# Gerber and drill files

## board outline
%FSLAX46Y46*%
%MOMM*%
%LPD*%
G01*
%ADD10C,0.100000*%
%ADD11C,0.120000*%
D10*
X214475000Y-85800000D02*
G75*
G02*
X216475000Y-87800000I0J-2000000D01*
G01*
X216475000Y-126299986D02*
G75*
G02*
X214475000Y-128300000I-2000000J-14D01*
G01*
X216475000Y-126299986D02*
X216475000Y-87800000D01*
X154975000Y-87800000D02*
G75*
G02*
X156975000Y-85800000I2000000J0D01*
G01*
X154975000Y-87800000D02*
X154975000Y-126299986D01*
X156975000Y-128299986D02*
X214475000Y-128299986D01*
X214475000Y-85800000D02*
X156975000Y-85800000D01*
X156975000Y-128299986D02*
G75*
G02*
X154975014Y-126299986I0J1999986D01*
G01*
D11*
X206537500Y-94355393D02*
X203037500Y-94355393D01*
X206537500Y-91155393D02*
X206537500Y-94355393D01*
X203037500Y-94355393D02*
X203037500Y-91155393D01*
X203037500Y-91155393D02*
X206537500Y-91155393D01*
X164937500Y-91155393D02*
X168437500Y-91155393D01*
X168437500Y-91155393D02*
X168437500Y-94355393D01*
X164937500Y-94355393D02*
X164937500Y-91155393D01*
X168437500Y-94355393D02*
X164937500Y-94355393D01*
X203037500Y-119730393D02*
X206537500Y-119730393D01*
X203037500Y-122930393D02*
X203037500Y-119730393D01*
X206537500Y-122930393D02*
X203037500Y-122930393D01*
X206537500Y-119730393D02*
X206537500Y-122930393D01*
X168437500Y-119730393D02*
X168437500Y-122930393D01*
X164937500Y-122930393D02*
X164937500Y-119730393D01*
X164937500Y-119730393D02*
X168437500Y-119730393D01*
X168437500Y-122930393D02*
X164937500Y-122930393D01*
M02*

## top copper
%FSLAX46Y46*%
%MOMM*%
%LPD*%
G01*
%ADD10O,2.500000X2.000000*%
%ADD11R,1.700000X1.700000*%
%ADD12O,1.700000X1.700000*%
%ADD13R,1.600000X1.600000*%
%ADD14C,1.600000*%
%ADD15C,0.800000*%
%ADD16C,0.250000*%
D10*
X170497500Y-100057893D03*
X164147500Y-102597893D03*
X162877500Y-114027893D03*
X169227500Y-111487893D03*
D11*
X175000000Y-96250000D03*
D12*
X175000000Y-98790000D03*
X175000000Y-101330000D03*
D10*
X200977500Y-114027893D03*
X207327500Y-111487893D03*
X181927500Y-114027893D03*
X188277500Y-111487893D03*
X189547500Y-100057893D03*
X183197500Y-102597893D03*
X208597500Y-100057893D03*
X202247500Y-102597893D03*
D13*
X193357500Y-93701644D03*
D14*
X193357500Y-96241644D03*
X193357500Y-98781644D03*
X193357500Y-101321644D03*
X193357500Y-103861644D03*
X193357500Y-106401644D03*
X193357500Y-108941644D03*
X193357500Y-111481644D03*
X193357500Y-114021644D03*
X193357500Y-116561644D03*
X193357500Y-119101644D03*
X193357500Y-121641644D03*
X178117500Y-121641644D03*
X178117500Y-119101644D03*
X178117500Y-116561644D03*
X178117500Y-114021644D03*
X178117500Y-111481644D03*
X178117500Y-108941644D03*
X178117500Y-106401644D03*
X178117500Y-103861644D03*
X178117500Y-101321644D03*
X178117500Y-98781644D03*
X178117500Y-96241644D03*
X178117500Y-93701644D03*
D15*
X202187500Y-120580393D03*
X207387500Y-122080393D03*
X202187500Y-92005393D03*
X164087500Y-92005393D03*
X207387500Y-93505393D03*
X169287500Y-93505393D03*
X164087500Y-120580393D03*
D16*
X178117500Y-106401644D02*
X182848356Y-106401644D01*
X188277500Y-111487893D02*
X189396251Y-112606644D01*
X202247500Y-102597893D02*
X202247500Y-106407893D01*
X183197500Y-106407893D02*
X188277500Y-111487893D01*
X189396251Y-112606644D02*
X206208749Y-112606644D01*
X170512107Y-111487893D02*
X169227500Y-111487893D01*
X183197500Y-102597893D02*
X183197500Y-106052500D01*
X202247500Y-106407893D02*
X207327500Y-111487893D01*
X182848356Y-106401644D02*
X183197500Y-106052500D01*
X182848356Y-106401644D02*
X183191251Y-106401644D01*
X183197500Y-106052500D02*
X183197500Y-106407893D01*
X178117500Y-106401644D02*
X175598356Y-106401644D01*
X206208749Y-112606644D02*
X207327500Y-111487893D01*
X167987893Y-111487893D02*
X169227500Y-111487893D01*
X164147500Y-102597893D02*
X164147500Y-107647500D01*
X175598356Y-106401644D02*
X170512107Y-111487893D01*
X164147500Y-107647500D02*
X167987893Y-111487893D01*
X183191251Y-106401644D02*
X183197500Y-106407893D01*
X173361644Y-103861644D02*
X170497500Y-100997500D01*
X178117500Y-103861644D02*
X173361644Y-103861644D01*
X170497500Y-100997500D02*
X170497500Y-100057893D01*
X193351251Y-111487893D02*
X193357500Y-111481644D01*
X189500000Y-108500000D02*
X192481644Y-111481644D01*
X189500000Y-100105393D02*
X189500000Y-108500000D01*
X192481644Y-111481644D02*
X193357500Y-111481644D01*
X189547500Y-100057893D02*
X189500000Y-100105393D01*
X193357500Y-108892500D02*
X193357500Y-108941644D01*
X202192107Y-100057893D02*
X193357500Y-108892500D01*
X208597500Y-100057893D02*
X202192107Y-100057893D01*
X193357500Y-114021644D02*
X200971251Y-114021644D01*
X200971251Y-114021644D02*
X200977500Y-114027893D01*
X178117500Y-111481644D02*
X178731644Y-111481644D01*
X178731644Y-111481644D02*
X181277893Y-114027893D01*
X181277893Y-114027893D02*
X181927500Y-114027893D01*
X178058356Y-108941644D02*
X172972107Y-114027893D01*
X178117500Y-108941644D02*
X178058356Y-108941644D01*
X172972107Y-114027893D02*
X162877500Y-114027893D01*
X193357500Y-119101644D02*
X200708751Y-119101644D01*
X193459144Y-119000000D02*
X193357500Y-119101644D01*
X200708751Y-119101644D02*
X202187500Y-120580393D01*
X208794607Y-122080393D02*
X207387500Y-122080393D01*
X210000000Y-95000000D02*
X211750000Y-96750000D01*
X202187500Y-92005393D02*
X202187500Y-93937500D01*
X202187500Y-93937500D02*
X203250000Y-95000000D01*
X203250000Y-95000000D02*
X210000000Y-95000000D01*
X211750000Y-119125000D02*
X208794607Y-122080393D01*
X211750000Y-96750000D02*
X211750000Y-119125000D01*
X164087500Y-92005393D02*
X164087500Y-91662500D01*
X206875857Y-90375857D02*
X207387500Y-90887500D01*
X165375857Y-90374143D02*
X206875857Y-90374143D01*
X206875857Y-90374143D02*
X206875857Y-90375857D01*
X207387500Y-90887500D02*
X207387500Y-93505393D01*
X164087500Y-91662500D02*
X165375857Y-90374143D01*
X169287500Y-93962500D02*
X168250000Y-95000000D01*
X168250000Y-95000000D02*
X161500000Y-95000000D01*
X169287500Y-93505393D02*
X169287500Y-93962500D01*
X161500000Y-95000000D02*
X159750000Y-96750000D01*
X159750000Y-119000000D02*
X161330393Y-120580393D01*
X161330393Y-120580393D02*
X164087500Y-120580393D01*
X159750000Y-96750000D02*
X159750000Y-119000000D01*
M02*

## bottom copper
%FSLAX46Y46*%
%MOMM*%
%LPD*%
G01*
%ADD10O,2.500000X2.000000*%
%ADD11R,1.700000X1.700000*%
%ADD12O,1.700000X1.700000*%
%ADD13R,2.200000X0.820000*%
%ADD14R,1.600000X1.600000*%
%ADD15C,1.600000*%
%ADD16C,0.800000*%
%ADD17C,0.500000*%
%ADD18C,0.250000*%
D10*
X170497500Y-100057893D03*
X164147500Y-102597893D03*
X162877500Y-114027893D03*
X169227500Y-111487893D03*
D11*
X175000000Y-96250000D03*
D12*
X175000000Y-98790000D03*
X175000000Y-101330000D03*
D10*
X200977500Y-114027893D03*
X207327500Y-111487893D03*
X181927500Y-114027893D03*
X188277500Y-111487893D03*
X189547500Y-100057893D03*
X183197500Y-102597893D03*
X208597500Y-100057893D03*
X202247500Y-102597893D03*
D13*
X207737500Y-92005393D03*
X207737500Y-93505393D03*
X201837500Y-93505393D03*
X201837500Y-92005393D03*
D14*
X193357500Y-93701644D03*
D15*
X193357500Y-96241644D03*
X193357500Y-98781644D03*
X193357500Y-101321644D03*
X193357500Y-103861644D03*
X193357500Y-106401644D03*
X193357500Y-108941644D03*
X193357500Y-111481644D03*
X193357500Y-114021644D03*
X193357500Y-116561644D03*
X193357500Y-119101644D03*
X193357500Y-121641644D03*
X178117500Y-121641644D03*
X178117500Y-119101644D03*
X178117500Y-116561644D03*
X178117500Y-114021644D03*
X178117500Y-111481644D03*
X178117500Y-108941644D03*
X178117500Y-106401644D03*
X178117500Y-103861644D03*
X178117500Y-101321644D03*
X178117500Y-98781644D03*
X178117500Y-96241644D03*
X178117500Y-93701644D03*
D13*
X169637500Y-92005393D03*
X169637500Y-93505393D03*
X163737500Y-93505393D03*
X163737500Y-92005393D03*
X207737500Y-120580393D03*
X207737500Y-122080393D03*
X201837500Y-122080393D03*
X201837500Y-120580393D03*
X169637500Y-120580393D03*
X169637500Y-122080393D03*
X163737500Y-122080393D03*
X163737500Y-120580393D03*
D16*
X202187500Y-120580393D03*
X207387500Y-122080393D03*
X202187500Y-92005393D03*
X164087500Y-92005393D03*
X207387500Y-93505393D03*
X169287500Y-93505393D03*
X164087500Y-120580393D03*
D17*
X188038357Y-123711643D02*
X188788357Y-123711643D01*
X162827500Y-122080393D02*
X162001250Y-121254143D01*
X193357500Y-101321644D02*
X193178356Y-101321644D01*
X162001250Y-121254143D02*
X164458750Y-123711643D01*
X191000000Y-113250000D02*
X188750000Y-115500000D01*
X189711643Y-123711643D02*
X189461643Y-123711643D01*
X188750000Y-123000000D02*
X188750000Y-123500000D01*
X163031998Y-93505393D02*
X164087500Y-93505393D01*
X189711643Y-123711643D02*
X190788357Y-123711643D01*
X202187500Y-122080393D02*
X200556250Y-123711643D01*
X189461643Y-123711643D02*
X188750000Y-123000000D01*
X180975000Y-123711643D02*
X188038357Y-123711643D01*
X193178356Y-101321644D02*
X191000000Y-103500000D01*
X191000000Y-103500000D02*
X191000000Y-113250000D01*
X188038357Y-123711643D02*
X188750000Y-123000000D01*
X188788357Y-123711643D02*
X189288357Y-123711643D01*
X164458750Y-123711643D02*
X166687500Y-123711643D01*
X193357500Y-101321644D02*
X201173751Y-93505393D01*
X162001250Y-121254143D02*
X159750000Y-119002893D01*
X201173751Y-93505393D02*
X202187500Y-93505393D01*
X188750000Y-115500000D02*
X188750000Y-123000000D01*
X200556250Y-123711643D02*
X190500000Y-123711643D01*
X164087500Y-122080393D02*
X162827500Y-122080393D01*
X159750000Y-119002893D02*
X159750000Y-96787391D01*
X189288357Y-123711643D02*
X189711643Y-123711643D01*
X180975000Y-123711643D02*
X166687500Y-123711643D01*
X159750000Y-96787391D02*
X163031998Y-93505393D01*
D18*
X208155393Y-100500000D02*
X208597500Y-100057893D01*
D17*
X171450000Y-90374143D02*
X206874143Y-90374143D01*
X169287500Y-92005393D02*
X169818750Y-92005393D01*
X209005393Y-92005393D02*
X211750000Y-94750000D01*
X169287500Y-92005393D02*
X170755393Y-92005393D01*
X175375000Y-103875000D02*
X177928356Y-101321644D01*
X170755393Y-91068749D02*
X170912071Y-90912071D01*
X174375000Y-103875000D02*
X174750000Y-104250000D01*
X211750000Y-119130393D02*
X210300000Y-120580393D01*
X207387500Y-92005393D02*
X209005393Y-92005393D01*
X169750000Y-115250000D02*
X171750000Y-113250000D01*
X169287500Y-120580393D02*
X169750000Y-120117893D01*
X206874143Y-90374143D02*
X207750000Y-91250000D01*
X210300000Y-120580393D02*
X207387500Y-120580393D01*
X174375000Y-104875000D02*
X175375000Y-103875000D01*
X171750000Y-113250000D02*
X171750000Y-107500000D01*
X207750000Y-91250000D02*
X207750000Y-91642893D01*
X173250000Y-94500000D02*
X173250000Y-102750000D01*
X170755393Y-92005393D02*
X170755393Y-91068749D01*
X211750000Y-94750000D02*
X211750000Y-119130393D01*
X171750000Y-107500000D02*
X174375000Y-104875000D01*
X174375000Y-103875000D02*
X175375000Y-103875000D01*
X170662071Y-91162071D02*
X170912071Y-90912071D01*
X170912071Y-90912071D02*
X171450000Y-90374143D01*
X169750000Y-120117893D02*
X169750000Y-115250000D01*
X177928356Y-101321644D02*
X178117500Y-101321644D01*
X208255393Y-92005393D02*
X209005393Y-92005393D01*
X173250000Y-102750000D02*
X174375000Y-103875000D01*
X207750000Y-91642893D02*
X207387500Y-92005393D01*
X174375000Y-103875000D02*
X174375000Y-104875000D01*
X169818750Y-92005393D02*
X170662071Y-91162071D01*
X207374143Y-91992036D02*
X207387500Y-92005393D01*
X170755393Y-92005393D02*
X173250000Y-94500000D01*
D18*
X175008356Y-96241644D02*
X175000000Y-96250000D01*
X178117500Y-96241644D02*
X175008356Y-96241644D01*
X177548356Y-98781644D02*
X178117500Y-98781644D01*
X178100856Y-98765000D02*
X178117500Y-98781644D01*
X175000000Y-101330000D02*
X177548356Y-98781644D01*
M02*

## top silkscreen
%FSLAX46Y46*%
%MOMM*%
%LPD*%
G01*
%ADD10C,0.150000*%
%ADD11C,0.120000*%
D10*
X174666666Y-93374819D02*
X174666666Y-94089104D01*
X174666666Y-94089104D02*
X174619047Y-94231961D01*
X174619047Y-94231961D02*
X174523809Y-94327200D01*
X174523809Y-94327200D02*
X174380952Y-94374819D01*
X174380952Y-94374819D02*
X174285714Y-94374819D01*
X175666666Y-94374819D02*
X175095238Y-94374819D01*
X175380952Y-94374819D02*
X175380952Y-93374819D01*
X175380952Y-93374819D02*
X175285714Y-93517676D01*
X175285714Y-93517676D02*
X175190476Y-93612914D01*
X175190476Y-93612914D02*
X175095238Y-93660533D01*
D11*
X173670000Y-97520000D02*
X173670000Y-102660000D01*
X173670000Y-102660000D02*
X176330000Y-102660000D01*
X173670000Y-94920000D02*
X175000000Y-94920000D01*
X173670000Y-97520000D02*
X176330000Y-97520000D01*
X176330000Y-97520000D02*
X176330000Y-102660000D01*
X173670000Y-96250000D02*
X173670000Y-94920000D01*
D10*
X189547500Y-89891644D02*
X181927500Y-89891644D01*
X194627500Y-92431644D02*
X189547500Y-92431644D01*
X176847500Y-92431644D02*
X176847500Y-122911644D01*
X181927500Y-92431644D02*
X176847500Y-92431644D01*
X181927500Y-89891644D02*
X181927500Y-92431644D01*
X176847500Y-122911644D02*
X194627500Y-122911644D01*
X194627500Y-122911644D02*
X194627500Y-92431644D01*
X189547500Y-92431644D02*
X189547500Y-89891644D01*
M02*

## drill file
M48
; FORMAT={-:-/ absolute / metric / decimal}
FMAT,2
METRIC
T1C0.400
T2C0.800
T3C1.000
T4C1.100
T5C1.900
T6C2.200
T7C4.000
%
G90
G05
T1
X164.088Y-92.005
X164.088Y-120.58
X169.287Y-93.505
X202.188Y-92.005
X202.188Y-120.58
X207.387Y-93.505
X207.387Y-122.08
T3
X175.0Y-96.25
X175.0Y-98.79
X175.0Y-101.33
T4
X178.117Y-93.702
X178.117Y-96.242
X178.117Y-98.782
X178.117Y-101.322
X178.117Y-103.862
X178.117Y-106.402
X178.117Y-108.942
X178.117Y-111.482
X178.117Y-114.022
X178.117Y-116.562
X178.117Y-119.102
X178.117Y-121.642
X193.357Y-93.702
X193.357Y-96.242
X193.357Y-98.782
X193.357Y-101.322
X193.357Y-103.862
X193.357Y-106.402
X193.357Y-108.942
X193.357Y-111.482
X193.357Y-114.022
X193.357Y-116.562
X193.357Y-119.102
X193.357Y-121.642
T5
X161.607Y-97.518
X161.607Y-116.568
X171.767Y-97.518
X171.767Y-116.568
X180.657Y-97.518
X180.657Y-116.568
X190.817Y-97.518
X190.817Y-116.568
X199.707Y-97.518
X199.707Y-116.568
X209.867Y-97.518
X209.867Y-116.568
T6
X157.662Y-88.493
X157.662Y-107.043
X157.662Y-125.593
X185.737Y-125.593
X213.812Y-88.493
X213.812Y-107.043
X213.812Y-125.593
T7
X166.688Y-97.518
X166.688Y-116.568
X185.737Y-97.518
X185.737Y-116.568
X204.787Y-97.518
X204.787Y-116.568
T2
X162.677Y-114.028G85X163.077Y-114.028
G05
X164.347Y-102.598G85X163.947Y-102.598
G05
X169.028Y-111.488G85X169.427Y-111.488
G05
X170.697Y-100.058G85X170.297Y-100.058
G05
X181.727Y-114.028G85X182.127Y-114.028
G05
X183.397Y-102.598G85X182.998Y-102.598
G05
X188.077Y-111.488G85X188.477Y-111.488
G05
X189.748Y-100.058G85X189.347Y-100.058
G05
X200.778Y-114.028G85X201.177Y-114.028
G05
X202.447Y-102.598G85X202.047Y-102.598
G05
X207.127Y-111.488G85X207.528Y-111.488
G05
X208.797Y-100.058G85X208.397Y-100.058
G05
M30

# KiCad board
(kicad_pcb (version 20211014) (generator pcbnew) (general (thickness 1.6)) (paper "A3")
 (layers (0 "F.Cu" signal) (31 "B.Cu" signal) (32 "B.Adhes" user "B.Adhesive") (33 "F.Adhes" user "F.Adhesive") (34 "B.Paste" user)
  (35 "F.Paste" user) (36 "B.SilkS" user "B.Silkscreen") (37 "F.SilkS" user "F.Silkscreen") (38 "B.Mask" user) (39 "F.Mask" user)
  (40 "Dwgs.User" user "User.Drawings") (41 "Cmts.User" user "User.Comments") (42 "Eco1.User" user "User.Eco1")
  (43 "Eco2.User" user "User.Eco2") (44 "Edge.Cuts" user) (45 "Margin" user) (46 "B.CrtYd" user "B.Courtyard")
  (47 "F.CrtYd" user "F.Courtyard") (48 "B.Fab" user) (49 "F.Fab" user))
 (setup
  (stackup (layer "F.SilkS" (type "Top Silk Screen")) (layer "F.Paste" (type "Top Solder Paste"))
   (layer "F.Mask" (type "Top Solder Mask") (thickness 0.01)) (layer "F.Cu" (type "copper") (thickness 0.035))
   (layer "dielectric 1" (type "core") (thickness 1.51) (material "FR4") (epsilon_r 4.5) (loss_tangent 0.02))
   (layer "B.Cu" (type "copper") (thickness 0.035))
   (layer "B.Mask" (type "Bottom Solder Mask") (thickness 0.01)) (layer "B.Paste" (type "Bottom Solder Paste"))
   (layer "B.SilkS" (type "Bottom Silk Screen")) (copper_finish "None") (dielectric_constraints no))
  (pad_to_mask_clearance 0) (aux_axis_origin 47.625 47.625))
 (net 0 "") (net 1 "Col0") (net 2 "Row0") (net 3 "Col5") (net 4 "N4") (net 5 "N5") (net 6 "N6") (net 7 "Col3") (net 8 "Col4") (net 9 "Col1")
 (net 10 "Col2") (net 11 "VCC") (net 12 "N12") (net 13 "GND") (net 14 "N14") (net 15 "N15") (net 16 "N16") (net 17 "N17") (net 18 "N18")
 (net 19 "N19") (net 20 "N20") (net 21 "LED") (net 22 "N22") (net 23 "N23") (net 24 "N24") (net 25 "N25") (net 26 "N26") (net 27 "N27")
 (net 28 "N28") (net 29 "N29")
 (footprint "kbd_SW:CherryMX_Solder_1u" (layer "F.Cu") (at 166.6875 97.517893 180)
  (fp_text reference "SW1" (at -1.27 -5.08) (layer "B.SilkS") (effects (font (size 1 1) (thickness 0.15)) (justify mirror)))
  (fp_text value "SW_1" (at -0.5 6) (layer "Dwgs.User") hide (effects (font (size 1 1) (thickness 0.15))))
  (pad "" np_thru_hole circle locked (at 0 0 270) (size 4 4) (drill 4) (layers *.Cu *.Mask))
  (pad "" np_thru_hole circle locked (at -5.08 0 270) (size 1.9 1.9) (drill 1.9) (layers *.Cu *.Mask))
  (pad "" np_thru_hole circle locked (at 5.08 0 270) (size 1.9 1.9) (drill 1.9) (layers *.Cu *.Mask))
  (pad "1" thru_hole oval locked (at -3.81 -2.54 180) (size 2.5 2) (drill oval 1.2 0.8) (layers *.Cu "B.Mask") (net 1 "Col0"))
  (pad "2" thru_hole oval locked (at 2.54 -5.08 180) (size 2.5 2) (drill oval 1.2 0.8) (layers *.Cu "B.Mask") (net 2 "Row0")))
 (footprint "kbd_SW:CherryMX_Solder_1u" (layer "F.Cu") (at 166.6875 116.567893)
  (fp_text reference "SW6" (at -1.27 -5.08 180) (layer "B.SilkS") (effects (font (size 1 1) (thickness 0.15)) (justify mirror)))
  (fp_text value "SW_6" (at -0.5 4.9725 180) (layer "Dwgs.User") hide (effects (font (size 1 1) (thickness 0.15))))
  (pad "" np_thru_hole circle locked (at 5.08 0 90) (size 1.9 1.9) (drill 1.9) (layers *.Cu *.Mask))
  (pad "" np_thru_hole circle locked (at 0 0 90) (size 4 4) (drill 4) (layers *.Cu *.Mask))
  (pad "" np_thru_hole circle locked (at -5.08 0 90) (size 1.9 1.9) (drill 1.9) (layers *.Cu *.Mask))
  (pad "1" thru_hole oval locked (at -3.81 -2.54) (size 2.5 2) (drill oval 1.2 0.8) (layers *.Cu "B.Mask") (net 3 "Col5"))
  (pad "2" thru_hole oval locked (at 2.54 -5.08) (size 2.5 2) (drill oval 1.2 0.8) (layers *.Cu "B.Mask") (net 2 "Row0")))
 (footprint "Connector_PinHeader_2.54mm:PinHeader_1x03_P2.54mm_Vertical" (layer "F.Cu") (at 175 96.25)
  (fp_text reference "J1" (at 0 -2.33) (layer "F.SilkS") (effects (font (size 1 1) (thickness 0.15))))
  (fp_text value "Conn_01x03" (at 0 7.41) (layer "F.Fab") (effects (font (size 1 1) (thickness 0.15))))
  (fp_line (start -1.33 1.27) (end -1.33 6.41) (layer "F.SilkS") (width 0.12))
  (fp_line (start -1.33 6.41) (end 1.33 6.41) (layer "F.SilkS") (width 0.12))
  (fp_line (start -1.33 -1.33) (end 0 -1.33) (layer "F.SilkS") (width 0.12))
  (fp_line (start -1.33 1.27) (end 1.33 1.27) (layer "F.SilkS") (width 0.12))
  (fp_line (start 1.33 1.27) (end 1.33 6.41) (layer "F.SilkS") (width 0.12))
  (fp_line (start -1.33 0) (end -1.33 -1.33) (layer "F.SilkS") (width 0.12))
  (pad "1" thru_hole rect (at 0 0) (size 1.7 1.7) (drill 1) (layers *.Cu *.Mask) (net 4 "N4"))
  (pad "2" thru_hole oval (at 0 2.54) (size 1.7 1.7) (drill 1) (layers *.Cu) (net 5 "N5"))
  (pad "3" thru_hole oval (at 0 5.08) (size 1.7 1.7) (drill 1) (layers *.Cu *.Mask) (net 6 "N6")))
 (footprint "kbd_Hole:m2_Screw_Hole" (layer "F.Cu") (at 213.8125 107.042893)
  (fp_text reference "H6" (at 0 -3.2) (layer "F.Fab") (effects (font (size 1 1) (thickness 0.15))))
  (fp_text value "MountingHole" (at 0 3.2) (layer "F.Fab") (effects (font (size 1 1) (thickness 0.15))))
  (pad "" np_thru_hole circle locked (at 0 0) (size 2.2 2.2) (drill 2.2) (layers *.Cu *.Mask)))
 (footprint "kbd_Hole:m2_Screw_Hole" (layer "F.Cu") (at 157.6625 88.492893) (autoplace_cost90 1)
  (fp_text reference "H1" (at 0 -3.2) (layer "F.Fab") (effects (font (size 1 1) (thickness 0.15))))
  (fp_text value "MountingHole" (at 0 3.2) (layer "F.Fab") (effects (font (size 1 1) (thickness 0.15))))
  (pad "" np_thru_hole circle locked (at 0 0) (size 2.2 2.2) (drill 2.2) (layers *.Cu *.Mask)))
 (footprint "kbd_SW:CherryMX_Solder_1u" (layer "F.Cu") (at 204.7875 116.567893)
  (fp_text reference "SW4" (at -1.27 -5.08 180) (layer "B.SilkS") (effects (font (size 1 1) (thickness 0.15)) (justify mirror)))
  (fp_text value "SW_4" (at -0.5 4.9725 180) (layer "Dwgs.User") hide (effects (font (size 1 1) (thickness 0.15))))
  (pad "" np_thru_hole circle locked (at 0 0 90) (size 4 4) (drill 4) (layers *.Cu *.Mask))
  (pad "" np_thru_hole circle locked (at 5.08 0 90) (size 1.9 1.9) (drill 1.9) (layers *.Cu *.Mask))
  (pad "" np_thru_hole circle locked (at -5.08 0 90) (size 1.9 1.9) (drill 1.9) (layers *.Cu *.Mask))
  (pad "1" thru_hole oval locked (at -3.81 -2.54) (size 2.5 2) (drill oval 1.2 0.8) (layers *.Cu "B.Mask") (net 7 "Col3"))
  (pad "2" thru_hole oval locked (at 2.54 -5.08) (size 2.5 2) (drill oval 1.2 0.8) (layers *.Cu "B.Mask") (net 2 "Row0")))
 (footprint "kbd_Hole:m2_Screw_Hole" (layer "F.Cu") (at 157.6625 107.042893)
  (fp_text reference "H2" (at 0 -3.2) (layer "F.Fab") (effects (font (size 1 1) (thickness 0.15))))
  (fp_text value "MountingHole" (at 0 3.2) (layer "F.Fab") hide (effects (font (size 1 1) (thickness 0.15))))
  (pad "" np_thru_hole circle locked (at 0 0) (size 2.2 2.2) (drill 2.2) (layers *.Cu *.Mask)))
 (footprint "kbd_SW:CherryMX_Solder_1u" (layer "F.Cu") (at 185.7375 116.567893)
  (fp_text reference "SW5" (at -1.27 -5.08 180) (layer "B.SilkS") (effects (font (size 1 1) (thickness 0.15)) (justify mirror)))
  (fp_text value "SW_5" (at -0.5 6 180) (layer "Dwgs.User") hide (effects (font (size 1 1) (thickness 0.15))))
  (pad "" np_thru_hole circle locked (at 0 0 90) (size 4 4) (drill 4) (layers *.Cu *.Mask))
  (pad "" np_thru_hole circle locked (at -5.08 0 90) (size 1.9 1.9) (drill 1.9) (layers *.Cu *.Mask))
  (pad "" np_thru_hole circle locked (at 5.08 0 90) (size 1.9 1.9) (drill 1.9) (layers *.Cu *.Mask))
  (pad "1" thru_hole oval locked (at -3.81 -2.54) (size 2.5 2) (drill oval 1.2 0.8) (layers *.Cu "B.Mask") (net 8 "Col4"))
  (pad "2" thru_hole oval locked (at 2.54 -5.08) (size 2.5 2) (drill oval 1.2 0.8) (layers *.Cu "B.Mask") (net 2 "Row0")))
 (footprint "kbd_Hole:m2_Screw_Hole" (layer "F.Cu") (at 185.7375 125.592893)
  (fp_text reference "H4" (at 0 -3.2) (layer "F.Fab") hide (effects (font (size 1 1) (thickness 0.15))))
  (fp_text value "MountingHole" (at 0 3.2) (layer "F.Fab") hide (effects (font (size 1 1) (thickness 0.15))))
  (pad "" np_thru_hole circle locked (at 0 0) (size 2.2 2.2) (drill 2.2) (layers *.Cu *.Mask)))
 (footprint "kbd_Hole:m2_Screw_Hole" (layer "F.Cu") (at 157.6625 125.592893)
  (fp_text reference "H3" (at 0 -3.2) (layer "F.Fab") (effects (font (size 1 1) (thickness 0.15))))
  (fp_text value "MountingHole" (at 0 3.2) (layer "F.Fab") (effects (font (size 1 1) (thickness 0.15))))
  (pad "" np_thru_hole circle locked (at 0 0) (size 2.2 2.2) (drill 2.2) (layers *.Cu *.Mask)))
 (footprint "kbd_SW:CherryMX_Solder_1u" (layer "F.Cu") (at 185.7375 97.517893 180)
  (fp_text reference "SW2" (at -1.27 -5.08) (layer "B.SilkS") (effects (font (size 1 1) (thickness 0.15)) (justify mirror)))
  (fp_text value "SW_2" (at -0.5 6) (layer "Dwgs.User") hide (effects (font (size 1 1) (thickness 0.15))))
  (pad "" np_thru_hole circle locked (at -5.08 0 270) (size 1.9 1.9) (drill 1.9) (layers *.Cu *.Mask))
  (pad "" np_thru_hole circle locked (at 5.08 0 270) (size 1.9 1.9) (drill 1.9) (layers *.Cu *.Mask))
  (pad "" np_thru_hole circle locked (at 0 0 270) (size 4 4) (drill 4) (layers *.Cu *.Mask))
  (pad "1" thru_hole oval locked (at -3.81 -2.54 180) (size 2.5 2) (drill oval 1.2 0.8) (layers *.Cu "B.Mask") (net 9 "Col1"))
  (pad "2" thru_hole oval locked (at 2.54 -5.08 180) (size 2.5 2) (drill oval 1.2 0.8) (layers *.Cu "B.Mask") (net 2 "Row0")))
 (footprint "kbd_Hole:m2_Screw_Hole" (layer "F.Cu") (at 213.8125 88.492893)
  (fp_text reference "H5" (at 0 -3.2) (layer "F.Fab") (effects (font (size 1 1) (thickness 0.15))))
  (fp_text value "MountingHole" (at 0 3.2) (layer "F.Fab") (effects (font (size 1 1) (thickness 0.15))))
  (pad "" np_thru_hole circle locked (at 0 0) (size 2.2 2.2) (drill 2.2) (layers *.Cu *.Mask)))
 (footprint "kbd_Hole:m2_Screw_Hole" (layer "F.Cu") (at 213.8125 125.592893)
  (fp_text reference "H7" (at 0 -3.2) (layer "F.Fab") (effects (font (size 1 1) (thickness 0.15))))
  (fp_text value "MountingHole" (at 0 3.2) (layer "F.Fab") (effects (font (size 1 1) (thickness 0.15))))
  (pad "" np_thru_hole circle locked (at 0 0) (size 2.2 2.2) (drill 2.2) (layers *.Cu *.Mask)))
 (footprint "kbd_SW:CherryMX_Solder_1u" (layer "F.Cu") (at 204.7875 97.517893 180)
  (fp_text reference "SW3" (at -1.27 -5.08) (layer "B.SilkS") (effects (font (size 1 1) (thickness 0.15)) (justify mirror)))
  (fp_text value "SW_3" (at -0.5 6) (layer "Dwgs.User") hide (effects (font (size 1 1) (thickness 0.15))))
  (pad "" np_thru_hole circle locked (at 0 0 270) (size 4 4) (drill 4) (layers *.Cu *.Mask))
  (pad "" np_thru_hole circle locked (at -5.08 0 270) (size 1.9 1.9) (drill 1.9) (layers *.Cu *.Mask))
  (pad "" np_thru_hole circle locked (at 5.08 0 270) (size 1.9 1.9) (drill 1.9) (layers *.Cu *.Mask))
  (pad "1" thru_hole oval locked (at -3.81 -2.54 180) (size 2.5 2) (drill oval 1.2 0.8) (layers *.Cu "B.Mask") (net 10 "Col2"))
  (pad "2" thru_hole oval locked (at 2.54 -5.08 180) (size 2.5 2) (drill oval 1.2 0.8) (layers *.Cu "B.Mask") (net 2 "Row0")))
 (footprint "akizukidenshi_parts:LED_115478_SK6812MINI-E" (layer "B.Cu") (at 204.7875 92.755393 180)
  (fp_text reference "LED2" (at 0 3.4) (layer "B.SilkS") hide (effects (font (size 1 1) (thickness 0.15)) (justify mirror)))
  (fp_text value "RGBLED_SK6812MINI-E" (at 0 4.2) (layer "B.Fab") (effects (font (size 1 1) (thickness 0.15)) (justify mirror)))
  (fp_line (start -1.75 -1.6) (end 1.75 -1.6) (layer "Edge.Cuts") (width 0.12))
  (fp_line (start -1.75 1.6) (end -1.75 -1.6) (layer "Edge.Cuts") (width 0.12))
  (fp_line (start 1.75 -1.6) (end 1.75 1.6) (layer "Edge.Cuts") (width 0.12))
  (fp_line (start 1.75 1.6) (end -1.75 1.6) (layer "Edge.Cuts") (width 0.12))
  (pad "1" smd rect (at -2.6 0.75 180) (size 2.2 0.82) (drill (offset -0.35 0)) (layers "B.Cu" "B.Paste" "B.Mask") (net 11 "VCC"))
  (pad "2" smd rect (at -2.6 -0.75 180) (size 2.2 0.82) (drill (offset -0.35 0)) (layers "B.Cu" "B.Paste" "B.Mask") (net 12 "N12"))
  (pad "3" smd rect (at 2.6 -0.75 180) (size 2.2 0.82) (drill (offset 0.35 0)) (layers "B.Cu" "B.Paste" "B.Mask") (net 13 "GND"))
  (pad "4" smd rect (at 2.6 0.75 180) (size 2.2 0.82) (drill (offset 0.35 0)) (layers "B.Cu" "B.Paste" "B.Mask") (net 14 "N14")))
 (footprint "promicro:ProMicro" (layer "B.Cu") (at 185.7375 107.671644 -90)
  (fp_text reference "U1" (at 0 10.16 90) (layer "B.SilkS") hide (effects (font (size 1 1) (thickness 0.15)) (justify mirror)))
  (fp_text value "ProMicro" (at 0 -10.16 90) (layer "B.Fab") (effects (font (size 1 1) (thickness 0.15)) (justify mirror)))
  (fp_line (start -17.78 -3.81) (end -17.78 3.81) (layer "F.SilkS") (width 0.15))
  (fp_line (start -15.24 -8.89) (end -15.24 -3.81) (layer "F.SilkS") (width 0.15))
  (fp_line (start -15.24 8.89) (end 15.24 8.89) (layer "F.SilkS") (width 0.15))
  (fp_line (start -15.24 3.81) (end -15.24 8.89) (layer "F.SilkS") (width 0.15))
  (fp_line (start -17.78 3.81) (end -15.24 3.81) (layer "F.SilkS") (width 0.15))
  (fp_line (start 15.24 8.89) (end 15.24 -8.89) (layer "F.SilkS") (width 0.15))
  (fp_line (start 15.24 -8.89) (end -15.24 -8.89) (layer "F.SilkS") (width 0.15))
  (fp_line (start -15.24 -3.81) (end -17.78 -3.81) (layer "F.SilkS") (width 0.15))
  (pad "1" thru_hole rect locked (at -13.97 -7.62 270) (size 1.6 1.6) (drill 1.1) (layers *.Cu *.Mask "B.SilkS") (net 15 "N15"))
  (pad "2" thru_hole circle locked (at -11.43 -7.62 270) (size 1.6 1.6) (drill 1.1) (layers *.Cu *.Mask "B.SilkS") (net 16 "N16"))
  (pad "3" thru_hole circle locked (at -8.89 -7.62 270) (size 1.6 1.6) (drill 1.1) (layers *.Cu *.Mask "B.SilkS") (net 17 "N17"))
  (pad "4" thru_hole circle locked (at -6.35 -7.62 270) (size 1.6 1.6) (drill 1.1) (layers *.Cu *.Mask "B.SilkS") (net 13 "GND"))
  (pad "5" thru_hole circle locked (at -3.81 -7.62 270) (size 1.6 1.6) (drill 1.1) (layers *.Cu *.Mask "B.SilkS") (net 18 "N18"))
  (pad "6" thru_hole circle locked (at -1.27 -7.62 270) (size 1.6 1.6) (drill 1.1) (layers *.Cu *.Mask "B.SilkS") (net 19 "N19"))
  (pad "7" thru_hole circle locked (at 1.27 -7.62 270) (size 1.6 1.6) (drill 1.1) (layers *.Cu *.Mask "B.SilkS") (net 10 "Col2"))
  (pad "8" thru_hole circle locked (at 3.81 -7.62 270) (size 1.6 1.6) (drill 1.1) (layers *.Cu *.Mask "B.SilkS") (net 9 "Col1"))
  (pad "9" thru_hole circle locked (at 6.35 -7.62 270) (size 1.6 1.6) (drill 1.1) (layers *.Cu *.Mask "B.SilkS") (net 7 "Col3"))
  (pad "10" thru_hole circle locked (at 8.89 -7.62 270) (size 1.6 1.6) (drill 1.1) (layers *.Cu *.Mask "B.SilkS") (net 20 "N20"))
  (pad "11" thru_hole circle locked (at 11.43 -7.62 270) (size 1.6 1.6) (drill 1.1) (layers *.Cu *.Mask "B.SilkS") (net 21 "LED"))
  (pad "12" thru_hole circle locked (at 13.97 -7.62 270) (size 1.6 1.6) (drill 1.1) (layers *.Cu *.Mask "B.SilkS") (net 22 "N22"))
  (pad "13" thru_hole circle locked (at 13.97 7.62 270) (size 1.6 1.6) (drill 1.1) (layers *.Cu *.Mask "B.SilkS") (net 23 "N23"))
  (pad "14" thru_hole circle locked (at 11.43 7.62 270) (size 1.6 1.6) (drill 1.1) (layers *.Cu *.Mask "B.SilkS") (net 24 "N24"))
  (pad "15" thru_hole circle locked (at 8.89 7.62 270) (size 1.6 1.6) (drill 1.1) (layers *.Cu *.Mask "B.SilkS") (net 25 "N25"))
  (pad "16" thru_hole circle locked (at 6.35 7.62 270) (size 1.6 1.6) (drill 1.1) (layers *.Cu *.Mask "B.SilkS") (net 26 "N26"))
  (pad "17" thru_hole circle locked (at 3.81 7.62 270) (size 1.6 1.6) (drill 1.1) (layers *.Cu *.Mask "B.SilkS") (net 8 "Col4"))
  (pad "18" thru_hole circle locked (at 1.27 7.62 270) (size 1.6 1.6) (drill 1.1) (layers *.Cu *.Mask "B.SilkS") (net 3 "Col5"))
  (pad "19" thru_hole circle locked (at -1.27 7.62 270) (size 1.6 1.6) (drill 1.1) (layers *.Cu *.Mask "B.SilkS") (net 2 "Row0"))
  (pad "20" thru_hole circle locked (at -3.81 7.62 270) (size 1.6 1.6) (drill 1.1) (layers *.Cu *.Mask "B.SilkS") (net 1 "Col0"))
  (pad "21" thru_hole circle locked (at -6.35 7.62 270) (size 1.6 1.6) (drill 1.1) (layers *.Cu *.Mask "B.SilkS") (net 11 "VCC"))
  (pad "22" thru_hole circle locked (at -8.89 7.62 270) (size 1.6 1.6) (drill 1.1) (layers *.Cu *.Mask "B.SilkS") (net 6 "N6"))
  (pad "23" thru_hole circle locked (at -11.43 7.62 270) (size 1.6 1.6) (drill 1.1) (layers *.Cu *.Mask "B.SilkS") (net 4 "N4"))
  (pad "24" thru_hole circle locked (at -13.97 7.62 270) (size 1.6 1.6) (drill 1.1) (layers *.Cu *.Mask "B.SilkS") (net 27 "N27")))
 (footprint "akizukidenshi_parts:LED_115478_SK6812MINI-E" (layer "B.Cu") (at 166.6875 92.755393 180)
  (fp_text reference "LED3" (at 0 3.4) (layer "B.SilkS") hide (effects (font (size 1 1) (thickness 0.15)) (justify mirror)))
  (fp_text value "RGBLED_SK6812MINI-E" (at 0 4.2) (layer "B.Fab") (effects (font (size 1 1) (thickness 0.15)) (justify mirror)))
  (fp_line (start 1.75 1.6) (end -1.75 1.6) (layer "Edge.Cuts") (width 0.12))
  (fp_line (start -1.75 1.6) (end -1.75 -1.6) (layer "Edge.Cuts") (width 0.12))
  (fp_line (start 1.75 -1.6) (end 1.75 1.6) (layer "Edge.Cuts") (width 0.12))
  (fp_line (start -1.75 -1.6) (end 1.75 -1.6) (layer "Edge.Cuts") (width 0.12))
  (pad "1" smd rect (at -2.6 0.75 180) (size 2.2 0.82) (drill (offset -0.35 0)) (layers "B.Cu" "B.Paste" "B.Mask") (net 11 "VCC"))
  (pad "2" smd rect (at -2.6 -0.75 180) (size 2.2 0.82) (drill (offset -0.35 0)) (layers "B.Cu" "B.Paste" "B.Mask") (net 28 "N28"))
  (pad "3" smd rect (at 2.6 -0.75 180) (size 2.2 0.82) (drill (offset 0.35 0)) (layers "B.Cu" "B.Paste" "B.Mask") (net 13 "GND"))
  (pad "4" smd rect (at 2.6 0.75 180) (size 2.2 0.82) (drill (offset 0.35 0)) (layers "B.Cu" "B.Paste" "B.Mask") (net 12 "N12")))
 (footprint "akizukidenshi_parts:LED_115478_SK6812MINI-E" (layer "B.Cu") (at 204.7875 121.330393 180)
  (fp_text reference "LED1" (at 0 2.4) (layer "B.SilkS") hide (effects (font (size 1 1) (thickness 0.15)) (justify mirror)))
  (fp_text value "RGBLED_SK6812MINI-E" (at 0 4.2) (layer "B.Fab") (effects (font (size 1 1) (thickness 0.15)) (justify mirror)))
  (fp_line (start 1.75 1.6) (end -1.75 1.6) (layer "Edge.Cuts") (width 0.12))
  (fp_line (start 1.75 -1.6) (end 1.75 1.6) (layer "Edge.Cuts") (width 0.12))
  (fp_line (start -1.75 -1.6) (end 1.75 -1.6) (layer "Edge.Cuts") (width 0.12))
  (fp_line (start -1.75 1.6) (end -1.75 -1.6) (layer "Edge.Cuts") (width 0.12))
  (pad "1" smd rect (at -2.6 0.75 180) (size 2.2 0.82) (drill (offset -0.35 0)) (layers "B.Cu" "B.Paste" "B.Mask") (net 11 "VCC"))
  (pad "2" smd rect (at -2.6 -0.75 180) (size 2.2 0.82) (drill (offset -0.35 0)) (layers "B.Cu" "B.Paste" "B.Mask") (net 14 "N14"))
  (pad "3" smd rect (at 2.6 -0.75 180) (size 2.2 0.82) (drill (offset 0.35 0)) (layers "B.Cu" "B.Paste" "B.Mask") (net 13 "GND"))
  (pad "4" smd rect (at 2.6 0.75 180) (size 2.2 0.82) (drill (offset 0.35 0)) (layers "B.Cu" "B.Paste" "B.Mask") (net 21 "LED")))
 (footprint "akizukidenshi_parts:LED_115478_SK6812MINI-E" (layer "B.Cu") (at 166.6875 121.330393 180)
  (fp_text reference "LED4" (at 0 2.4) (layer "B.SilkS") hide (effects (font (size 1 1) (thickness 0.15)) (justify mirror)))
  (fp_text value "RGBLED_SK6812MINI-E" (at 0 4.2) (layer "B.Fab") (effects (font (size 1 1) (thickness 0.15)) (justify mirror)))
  (fp_line (start -1.75 1.6) (end -1.75 -1.6) (layer "Edge.Cuts") (width 0.12))
  (fp_line (start 1.75 -1.6) (end 1.75 1.6) (layer "Edge.Cuts") (width 0.12))
  (fp_line (start 1.75 1.6) (end -1.75 1.6) (layer "Edge.Cuts") (width 0.12))
  (fp_line (start -1.75 -1.6) (end 1.75 -1.6) (layer "Edge.Cuts") (width 0.12))
  (pad "1" smd rect (at -2.6 0.75 180) (size 2.2 0.82) (drill (offset -0.35 0)) (layers "B.Cu" "B.Paste" "B.Mask") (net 11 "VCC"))
  (pad "2" smd rect (at -2.6 -0.75 180) (size 2.2 0.82) (drill (offset -0.35 0)) (layers "B.Cu" "B.Paste" "B.Mask") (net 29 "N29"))
  (pad "3" smd rect (at 2.6 -0.75 180) (size 2.2 0.82) (drill (offset 0.35 0)) (layers "B.Cu" "B.Paste" "B.Mask") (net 13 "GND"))
  (pad "4" smd rect (at 2.6 0.75 180) (size 2.2 0.82) (drill (offset 0.35 0)) (layers "B.Cu" "B.Paste" "B.Mask") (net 28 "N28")))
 (gr_arc (start 214.475 85.8) (mid 215.889214 86.385786) (end 216.475 87.8) (layer "Edge.Cuts") (width 0.1))
 (gr_arc (start 216.475 126.299986) (mid 215.889216 127.714202) (end 214.475 128.299986) (layer "Edge.Cuts") (width 0.1))
 (gr_line (start 216.475 126.299986) (end 216.475 87.8) (layer "Edge.Cuts") (width 0.1))
 (gr_arc (start 154.975 87.8) (mid 155.560786 86.385786) (end 156.975 85.8) (layer "Edge.Cuts") (width 0.1))
 (gr_line (start 154.975 87.8) (end 154.975 126.299986) (layer "Edge.Cuts") (width 0.1))
 (gr_line (start 156.975 128.299986) (end 214.475 128.299986) (layer "Edge.Cuts") (width 0.1))
 (gr_line (start 214.475 85.8) (end 156.975 85.8) (layer "Edge.Cuts") (width 0.1))
 (gr_arc (start 156.975 128.299986) (mid 155.560784 127.714202) (end 154.975 126.299986) (layer "Edge.Cuts") (width 0.1))
 (segment (start 188.038357 123.711643) (end 188.788357 123.711643) (width 0.5) (layer "B.Cu") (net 13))
 (segment (start 162.8275 122.080393) (end 162.00125 121.254143) (width 0.5) (layer "B.Cu") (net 13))
 (segment (start 193.3575 101.321644) (end 193.178356 101.321644) (width 0.5) (layer "B.Cu") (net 13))
 (segment (start 162.00125 121.254143) (end 164.45875 123.711643) (width 0.5) (layer "B.Cu") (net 13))
 (segment (start 191 113.25) (end 188.75 115.5) (width 0.5) (layer "B.Cu") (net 13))
 (segment (start 189.711643 123.711643) (end 189.461643 123.711643) (width 0.5) (layer "B.Cu") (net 13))
 (segment (start 188.75 123) (end 188.75 123.5) (width 0.5) (layer "B.Cu") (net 13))
 (segment (start 163.031998 93.505393) (end 164.0875 93.505393) (width 0.5) (layer "B.Cu") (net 13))
 (segment (start 189.711643 123.711643) (end 190.788357 123.711643) (width 0.5) (layer "B.Cu") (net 13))
 (segment (start 202.1875 122.080393) (end 200.55625 123.711643) (width 0.5) (layer "B.Cu") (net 13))
 (segment (start 189.461643 123.711643) (end 188.75 123) (width 0.5) (layer "B.Cu") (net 13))
 (segment (start 180.975 123.711643) (end 188.038357 123.711643) (width 0.5) (layer "B.Cu") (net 13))
 (segment (start 193.178356 101.321644) (end 191 103.5) (width 0.5) (layer "B.Cu") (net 13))
 (segment (start 191 103.5) (end 191 113.25) (width 0.5) (layer "B.Cu") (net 13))
 (segment (start 188.038357 123.711643) (end 188.75 123) (width 0.5) (layer "B.Cu") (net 13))
 (segment (start 188.788357 123.711643) (end 189.288357 123.711643) (width 0.5) (layer "B.Cu") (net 13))
 (segment (start 164.45875 123.711643) (end 166.6875 123.711643) (width 0.5) (layer "B.Cu") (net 13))
 (segment (start 193.3575 101.321644) (end 201.173751 93.505393) (width 0.5) (layer "B.Cu") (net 13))
 (segment (start 162.00125 121.254143) (end 159.75 119.002893) (width 0.5) (layer "B.Cu") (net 13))
 (segment (start 201.173751 93.505393) (end 202.1875 93.505393) (width 0.5) (layer "B.Cu") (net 13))
 (segment (start 188.75 115.5) (end 188.75 123) (width 0.5) (layer "B.Cu") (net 13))
 (segment (start 200.55625 123.711643) (end 190.5 123.711643) (width 0.5) (layer "B.Cu") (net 13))
 (segment (start 164.0875 122.080393) (end 162.8275 122.080393) (width 0.5) (layer "B.Cu") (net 13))
 (segment (start 159.75 119.002893) (end 159.75 96.787391) (width 0.5) (layer "B.Cu") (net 13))
 (segment (start 189.288357 123.711643) (end 189.711643 123.711643) (width 0.5) (layer "B.Cu") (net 13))
 (segment (start 180.975 123.711643) (end 166.6875 123.711643) (width 0.5) (layer "B.Cu") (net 13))
 (segment (start 159.75 96.787391) (end 163.031998 93.505393) (width 0.5) (layer "B.Cu") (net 13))
 (segment (start 178.1175 106.401644) (end 182.848356 106.401644) (width 0.25) (layer "F.Cu") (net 2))
 (segment (start 188.2775 111.487893) (end 189.396251 112.606644) (width 0.25) (layer "F.Cu") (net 2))
 (segment (start 202.2475 102.597893) (end 202.2475 106.407893) (width 0.25) (layer "F.Cu") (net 2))
 (segment (start 183.1975 106.407893) (end 188.2775 111.487893) (width 0.25) (layer "F.Cu") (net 2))
 (segment (start 189.396251 112.606644) (end 206.208749 112.606644) (width 0.25) (layer "F.Cu") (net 2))
 (segment (start 170.512107 111.487893) (end 169.2275 111.487893) (width 0.25) (layer "F.Cu") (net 2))
 (segment (start 183.1975 102.597893) (end 183.1975 106.0525) (width 0.25) (layer "F.Cu") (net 2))
 (segment (start 202.2475 106.407893) (end 207.3275 111.487893) (width 0.25) (layer "F.Cu") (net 2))
 (segment (start 182.848356 106.401644) (end 183.1975 106.0525) (width 0.25) (layer "F.Cu") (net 2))
 (segment (start 182.848356 106.401644) (end 183.191251 106.401644) (width 0.25) (layer "F.Cu") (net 2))
 (segment (start 183.1975 106.0525) (end 183.1975 106.407893) (width 0.25) (layer "F.Cu") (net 2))
 (segment (start 178.1175 106.401644) (end 175.598356 106.401644) (width 0.25) (layer "F.Cu") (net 2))
 (segment (start 206.208749 112.606644) (end 207.3275 111.487893) (width 0.25) (layer "F.Cu") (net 2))
 (segment (start 167.987893 111.487893) (end 169.2275 111.487893) (width 0.25) (layer "F.Cu") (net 2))
 (segment (start 164.1475 102.597893) (end 164.1475 107.6475) (width 0.25) (layer "F.Cu") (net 2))
 (segment (start 175.598356 106.401644) (end 170.512107 111.487893) (width 0.25) (layer "F.Cu") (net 2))
 (segment (start 164.1475 107.6475) (end 167.987893 111.487893) (width 0.25) (layer "F.Cu") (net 2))
 (segment (start 183.191251 106.401644) (end 183.1975 106.407893) (width 0.25) (layer "F.Cu") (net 2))
 (segment (start 173.361644 103.861644) (end 170.4975 100.9975) (width 0.25) (layer "F.Cu") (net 1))
 (segment (start 178.1175 103.861644) (end 173.361644 103.861644) (width 0.25) (layer "F.Cu") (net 1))
 (segment (start 170.4975 100.9975) (end 170.4975 100.057893) (width 0.25) (layer "F.Cu") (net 1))
 (segment (start 193.351251 111.487893) (end 193.3575 111.481644) (width 0.25) (layer "F.Cu") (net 9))
 (segment (start 189.5 108.5) (end 192.481644 111.481644) (width 0.25) (layer "F.Cu") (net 9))
 (segment (start 189.5 100.105393) (end 189.5 108.5) (width 0.25) (layer "F.Cu") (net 9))
 (segment (start 192.481644 111.481644) (end 193.3575 111.481644) (width 0.25) (layer "F.Cu") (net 9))
 (segment (start 189.5475 100.057893) (end 189.5 100.105393) (width 0.25) (layer "F.Cu") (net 9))
 (segment (start 193.3575 108.8925) (end 193.3575 108.941644) (width 0.25) (layer "F.Cu") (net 10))
 (segment (start 202.192107 100.057893) (end 193.3575 108.8925) (width 0.25) (layer "F.Cu") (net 10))
 (segment (start 208.5975 100.057893) (end 202.192107 100.057893) (width 0.25) (layer "F.Cu") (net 10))
 (segment (start 208.155393 100.5) (end 208.5975 100.057893) (width 0.25) (layer "B.Cu") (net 10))
 (segment (start 193.3575 114.021644) (end 200.971251 114.021644) (width 0.25) (layer "F.Cu") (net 7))
 (segment (start 200.971251 114.021644) (end 200.9775 114.027893) (width 0.25) (layer "F.Cu") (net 7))
 (segment (start 178.1175 111.481644) (end 178.731644 111.481644) (width 0.25) (layer "F.Cu") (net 8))
 (segment (start 178.731644 111.481644) (end 181.277893 114.027893) (width 0.25) (layer "F.Cu") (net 8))
 (segment (start 181.277893 114.027893) (end 181.9275 114.027893) (width 0.25) (layer "F.Cu") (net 8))
 (segment (start 178.058356 108.941644) (end 172.972107 114.027893) (width 0.25) (layer "F.Cu") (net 3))
 (segment (start 178.1175 108.941644) (end 178.058356 108.941644) (width 0.25) (layer "F.Cu") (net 3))
 (segment (start 172.972107 114.027893) (end 162.8775 114.027893) (width 0.25) (layer "F.Cu") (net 3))
 (segment (start 171.45 90.374143) (end 206.874143 90.374143) (width 0.5) (layer "B.Cu") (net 11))
 (segment (start 169.2875 92.005393) (end 169.81875 92.005393) (width 0.5) (layer "B.Cu") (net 11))
 (segment (start 209.005393 92.005393) (end 211.75 94.75) (width 0.5) (layer "B.Cu") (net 11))
 (segment (start 169.2875 92.005393) (end 170.755393 92.005393) (width 0.5) (layer "B.Cu") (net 11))
 (segment (start 175.375 103.875) (end 177.928356 101.321644) (width 0.5) (layer "B.Cu") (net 11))
 (segment (start 170.755393 91.068749) (end 170.912071 90.912071) (width 0.5) (layer "B.Cu") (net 11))
 (segment (start 174.375 103.875) (end 174.75 104.25) (width 0.5) (layer "B.Cu") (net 11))
 (segment (start 211.75 119.130393) (end 210.3 120.580393) (width 0.5) (layer "B.Cu") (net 11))
 (segment (start 207.3875 92.005393) (end 209.005393 92.005393) (width 0.5) (layer "B.Cu") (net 11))
 (segment (start 169.75 115.25) (end 171.75 113.25) (width 0.5) (layer "B.Cu") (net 11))
 (segment (start 169.2875 120.580393) (end 169.75 120.117893) (width 0.5) (layer "B.Cu") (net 11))
 (segment (start 206.874143 90.374143) (end 207.75 91.25) (width 0.5) (layer "B.Cu") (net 11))
 (segment (start 210.3 120.580393) (end 207.3875 120.580393) (width 0.5) (layer "B.Cu") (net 11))
 (segment (start 174.375 104.875) (end 175.375 103.875) (width 0.5) (layer "B.Cu") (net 11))
 (segment (start 171.75 113.25) (end 171.75 107.5) (width 0.5) (layer "B.Cu") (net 11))
 (segment (start 207.75 91.25) (end 207.75 91.642893) (width 0.5) (layer "B.Cu") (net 11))
 (segment (start 173.25 94.5) (end 173.25 102.75) (width 0.5) (layer "B.Cu") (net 11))
 (segment (start 170.755393 92.005393) (end 170.755393 91.068749) (width 0.5) (layer "B.Cu") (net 11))
 (segment (start 211.75 94.75) (end 211.75 119.130393) (width 0.5) (layer "B.Cu") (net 11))
 (segment (start 171.75 107.5) (end 174.375 104.875) (width 0.5) (layer "B.Cu") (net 11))
 (segment (start 174.375 103.875) (end 175.375 103.875) (width 0.5) (layer "B.Cu") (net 11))
 (segment (start 170.662071 91.162071) (end 170.912071 90.912071) (width 0.5) (layer "B.Cu") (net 11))
 (segment (start 170.912071 90.912071) (end 171.45 90.374143) (width 0.5) (layer "B.Cu") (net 11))
 (segment (start 169.75 120.117893) (end 169.75 115.25) (width 0.5) (layer "B.Cu") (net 11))
 (segment (start 177.928356 101.321644) (end 178.1175 101.321644) (width 0.5) (layer "B.Cu") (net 11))
 (segment (start 208.255393 92.005393) (end 209.005393 92.005393) (width 0.5) (layer "B.Cu") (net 11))
 (segment (start 173.25 102.75) (end 174.375 103.875) (width 0.5) (layer "B.Cu") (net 11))
 (segment (start 207.75 91.642893) (end 207.3875 92.005393) (width 0.5) (layer "B.Cu") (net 11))
 (segment (start 174.375 103.875) (end 174.375 104.875) (width 0.5) (layer "B.Cu") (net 11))
 (segment (start 169.81875 92.005393) (end 170.662071 91.162071) (width 0.5) (layer "B.Cu") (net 11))
 (segment (start 207.374143 91.992036) (end 207.3875 92.005393) (width 0.5) (layer "B.Cu") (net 11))
 (segment (start 170.755393 92.005393) (end 173.25 94.5) (width 0.5) (layer "B.Cu") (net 11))
 (segment (start 193.3575 119.101644) (end 200.708751 119.101644) (width 0.25) (layer "F.Cu") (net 21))
 (segment (start 193.459144 119) (end 193.3575 119.101644) (width 0.25) (layer "F.Cu") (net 21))
 (segment (start 200.708751 119.101644) (end 202.1875 120.580393) (width 0.25) (layer "F.Cu") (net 21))
 (via (at 202.1875 120.580393) (size 0.8) (drill 0.4) (layers "F.Cu" "B.Cu") (remove_unused_layers) (keep_end_layers) (free) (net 21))
 (segment (start 208.794607 122.080393) (end 207.3875 122.080393) (width 0.25) (layer "F.Cu") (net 14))
 (segment (start 210 95) (end 211.75 96.75) (width 0.25) (layer "F.Cu") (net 14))
 (segment (start 202.1875 92.005393) (end 202.1875 93.9375) (width 0.25) (layer "F.Cu") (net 14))
 (segment (start 202.1875 93.9375) (end 203.25 95) (width 0.25) (layer "F.Cu") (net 14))
 (segment (start 203.25 95) (end 210 95) (width 0.25) (layer "F.Cu") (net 14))
 (segment (start 211.75 119.125) (end 208.794607 122.080393) (width 0.25) (layer "F.Cu") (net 14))
 (segment (start 211.75 96.75) (end 211.75 119.125) (width 0.25) (layer "F.Cu") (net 14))
 (via (at 207.3875 122.080393) (size 0.8) (drill 0.4) (layers "F.Cu" "B.Cu") (free) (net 14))
 (via (at 202.1875 92.005393) (size 0.8) (drill 0.4) (layers "F.Cu" "B.Cu") (free) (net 14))
 (segment (start 164.0875 92.005393) (end 164.0875 91.6625) (width 0.25) (layer "F.Cu") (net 12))
 (segment (start 206.875857 90.375857) (end 207.3875 90.8875) (width 0.25) (layer "F.Cu") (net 12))
 (segment (start 165.375857 90.374143) (end 206.875857 90.374143) (width 0.25) (layer "F.Cu") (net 12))
 (segment (start 206.875857 90.374143) (end 206.875857 90.375857) (width 0.25) (layer "F.Cu") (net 12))
 (segment (start 207.3875 90.8875) (end 207.3875 93.505393) (width 0.25) (layer "F.Cu") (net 12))
 (segment (start 164.0875 91.6625) (end 165.375857 90.374143) (width 0.25) (layer "F.Cu") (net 12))
 (via (at 164.0875 92.005393) (size 0.8) (drill 0.4) (layers "F.Cu" "B.Cu") (free) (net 12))
 (via (at 207.3875 93.505393) (size 0.8) (drill 0.4) (layers "F.Cu" "B.Cu") (free) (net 12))
 (segment (start 169.2875 93.9625) (end 168.25 95) (width 0.25) (layer "F.Cu") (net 28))
 (segment (start 168.25 95) (end 161.5 95) (width 0.25) (layer "F.Cu") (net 28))
 (segment (start 169.2875 93.505393) (end 169.2875 93.9625) (width 0.25) (layer "F.Cu") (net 28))
 (segment (start 161.5 95) (end 159.75 96.75) (width 0.25) (layer "F.Cu") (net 28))
 (segment (start 159.75 119) (end 161.330393 120.580393) (width 0.25) (layer "F.Cu") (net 28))
 (segment (start 161.330393 120.580393) (end 164.0875 120.580393) (width 0.25) (layer "F.Cu") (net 28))
 (segment (start 159.75 96.75) (end 159.75 119) (width 0.25) (layer "F.Cu") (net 28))
 (via (at 169.2875 93.505393) (size 0.8) (drill 0.4) (layers "F.Cu" "B.Cu") (free) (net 28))
 (via (at 164.0875 120.580393) (size 0.8) (drill 0.4) (layers "F.Cu" "B.Cu") (free) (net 28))
 (segment (start 175.008356 96.241644) (end 175 96.25) (width 0.25) (layer "B.Cu") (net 4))
 (segment (start 178.1175 96.241644) (end 175.008356 96.241644) (width 0.25) (layer "B.Cu") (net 4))
 (segment (start 177.548356 98.781644) (end 178.1175 98.781644) (width 0.25) (layer "B.Cu") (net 6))
 (segment (start 178.100856 98.765) (end 178.1175 98.781644) (width 0.25) (layer "B.Cu") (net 6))
 (segment (start 175 101.33) (end 177.548356 98.781644) (width 0.25) (layer "B.Cu") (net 6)))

